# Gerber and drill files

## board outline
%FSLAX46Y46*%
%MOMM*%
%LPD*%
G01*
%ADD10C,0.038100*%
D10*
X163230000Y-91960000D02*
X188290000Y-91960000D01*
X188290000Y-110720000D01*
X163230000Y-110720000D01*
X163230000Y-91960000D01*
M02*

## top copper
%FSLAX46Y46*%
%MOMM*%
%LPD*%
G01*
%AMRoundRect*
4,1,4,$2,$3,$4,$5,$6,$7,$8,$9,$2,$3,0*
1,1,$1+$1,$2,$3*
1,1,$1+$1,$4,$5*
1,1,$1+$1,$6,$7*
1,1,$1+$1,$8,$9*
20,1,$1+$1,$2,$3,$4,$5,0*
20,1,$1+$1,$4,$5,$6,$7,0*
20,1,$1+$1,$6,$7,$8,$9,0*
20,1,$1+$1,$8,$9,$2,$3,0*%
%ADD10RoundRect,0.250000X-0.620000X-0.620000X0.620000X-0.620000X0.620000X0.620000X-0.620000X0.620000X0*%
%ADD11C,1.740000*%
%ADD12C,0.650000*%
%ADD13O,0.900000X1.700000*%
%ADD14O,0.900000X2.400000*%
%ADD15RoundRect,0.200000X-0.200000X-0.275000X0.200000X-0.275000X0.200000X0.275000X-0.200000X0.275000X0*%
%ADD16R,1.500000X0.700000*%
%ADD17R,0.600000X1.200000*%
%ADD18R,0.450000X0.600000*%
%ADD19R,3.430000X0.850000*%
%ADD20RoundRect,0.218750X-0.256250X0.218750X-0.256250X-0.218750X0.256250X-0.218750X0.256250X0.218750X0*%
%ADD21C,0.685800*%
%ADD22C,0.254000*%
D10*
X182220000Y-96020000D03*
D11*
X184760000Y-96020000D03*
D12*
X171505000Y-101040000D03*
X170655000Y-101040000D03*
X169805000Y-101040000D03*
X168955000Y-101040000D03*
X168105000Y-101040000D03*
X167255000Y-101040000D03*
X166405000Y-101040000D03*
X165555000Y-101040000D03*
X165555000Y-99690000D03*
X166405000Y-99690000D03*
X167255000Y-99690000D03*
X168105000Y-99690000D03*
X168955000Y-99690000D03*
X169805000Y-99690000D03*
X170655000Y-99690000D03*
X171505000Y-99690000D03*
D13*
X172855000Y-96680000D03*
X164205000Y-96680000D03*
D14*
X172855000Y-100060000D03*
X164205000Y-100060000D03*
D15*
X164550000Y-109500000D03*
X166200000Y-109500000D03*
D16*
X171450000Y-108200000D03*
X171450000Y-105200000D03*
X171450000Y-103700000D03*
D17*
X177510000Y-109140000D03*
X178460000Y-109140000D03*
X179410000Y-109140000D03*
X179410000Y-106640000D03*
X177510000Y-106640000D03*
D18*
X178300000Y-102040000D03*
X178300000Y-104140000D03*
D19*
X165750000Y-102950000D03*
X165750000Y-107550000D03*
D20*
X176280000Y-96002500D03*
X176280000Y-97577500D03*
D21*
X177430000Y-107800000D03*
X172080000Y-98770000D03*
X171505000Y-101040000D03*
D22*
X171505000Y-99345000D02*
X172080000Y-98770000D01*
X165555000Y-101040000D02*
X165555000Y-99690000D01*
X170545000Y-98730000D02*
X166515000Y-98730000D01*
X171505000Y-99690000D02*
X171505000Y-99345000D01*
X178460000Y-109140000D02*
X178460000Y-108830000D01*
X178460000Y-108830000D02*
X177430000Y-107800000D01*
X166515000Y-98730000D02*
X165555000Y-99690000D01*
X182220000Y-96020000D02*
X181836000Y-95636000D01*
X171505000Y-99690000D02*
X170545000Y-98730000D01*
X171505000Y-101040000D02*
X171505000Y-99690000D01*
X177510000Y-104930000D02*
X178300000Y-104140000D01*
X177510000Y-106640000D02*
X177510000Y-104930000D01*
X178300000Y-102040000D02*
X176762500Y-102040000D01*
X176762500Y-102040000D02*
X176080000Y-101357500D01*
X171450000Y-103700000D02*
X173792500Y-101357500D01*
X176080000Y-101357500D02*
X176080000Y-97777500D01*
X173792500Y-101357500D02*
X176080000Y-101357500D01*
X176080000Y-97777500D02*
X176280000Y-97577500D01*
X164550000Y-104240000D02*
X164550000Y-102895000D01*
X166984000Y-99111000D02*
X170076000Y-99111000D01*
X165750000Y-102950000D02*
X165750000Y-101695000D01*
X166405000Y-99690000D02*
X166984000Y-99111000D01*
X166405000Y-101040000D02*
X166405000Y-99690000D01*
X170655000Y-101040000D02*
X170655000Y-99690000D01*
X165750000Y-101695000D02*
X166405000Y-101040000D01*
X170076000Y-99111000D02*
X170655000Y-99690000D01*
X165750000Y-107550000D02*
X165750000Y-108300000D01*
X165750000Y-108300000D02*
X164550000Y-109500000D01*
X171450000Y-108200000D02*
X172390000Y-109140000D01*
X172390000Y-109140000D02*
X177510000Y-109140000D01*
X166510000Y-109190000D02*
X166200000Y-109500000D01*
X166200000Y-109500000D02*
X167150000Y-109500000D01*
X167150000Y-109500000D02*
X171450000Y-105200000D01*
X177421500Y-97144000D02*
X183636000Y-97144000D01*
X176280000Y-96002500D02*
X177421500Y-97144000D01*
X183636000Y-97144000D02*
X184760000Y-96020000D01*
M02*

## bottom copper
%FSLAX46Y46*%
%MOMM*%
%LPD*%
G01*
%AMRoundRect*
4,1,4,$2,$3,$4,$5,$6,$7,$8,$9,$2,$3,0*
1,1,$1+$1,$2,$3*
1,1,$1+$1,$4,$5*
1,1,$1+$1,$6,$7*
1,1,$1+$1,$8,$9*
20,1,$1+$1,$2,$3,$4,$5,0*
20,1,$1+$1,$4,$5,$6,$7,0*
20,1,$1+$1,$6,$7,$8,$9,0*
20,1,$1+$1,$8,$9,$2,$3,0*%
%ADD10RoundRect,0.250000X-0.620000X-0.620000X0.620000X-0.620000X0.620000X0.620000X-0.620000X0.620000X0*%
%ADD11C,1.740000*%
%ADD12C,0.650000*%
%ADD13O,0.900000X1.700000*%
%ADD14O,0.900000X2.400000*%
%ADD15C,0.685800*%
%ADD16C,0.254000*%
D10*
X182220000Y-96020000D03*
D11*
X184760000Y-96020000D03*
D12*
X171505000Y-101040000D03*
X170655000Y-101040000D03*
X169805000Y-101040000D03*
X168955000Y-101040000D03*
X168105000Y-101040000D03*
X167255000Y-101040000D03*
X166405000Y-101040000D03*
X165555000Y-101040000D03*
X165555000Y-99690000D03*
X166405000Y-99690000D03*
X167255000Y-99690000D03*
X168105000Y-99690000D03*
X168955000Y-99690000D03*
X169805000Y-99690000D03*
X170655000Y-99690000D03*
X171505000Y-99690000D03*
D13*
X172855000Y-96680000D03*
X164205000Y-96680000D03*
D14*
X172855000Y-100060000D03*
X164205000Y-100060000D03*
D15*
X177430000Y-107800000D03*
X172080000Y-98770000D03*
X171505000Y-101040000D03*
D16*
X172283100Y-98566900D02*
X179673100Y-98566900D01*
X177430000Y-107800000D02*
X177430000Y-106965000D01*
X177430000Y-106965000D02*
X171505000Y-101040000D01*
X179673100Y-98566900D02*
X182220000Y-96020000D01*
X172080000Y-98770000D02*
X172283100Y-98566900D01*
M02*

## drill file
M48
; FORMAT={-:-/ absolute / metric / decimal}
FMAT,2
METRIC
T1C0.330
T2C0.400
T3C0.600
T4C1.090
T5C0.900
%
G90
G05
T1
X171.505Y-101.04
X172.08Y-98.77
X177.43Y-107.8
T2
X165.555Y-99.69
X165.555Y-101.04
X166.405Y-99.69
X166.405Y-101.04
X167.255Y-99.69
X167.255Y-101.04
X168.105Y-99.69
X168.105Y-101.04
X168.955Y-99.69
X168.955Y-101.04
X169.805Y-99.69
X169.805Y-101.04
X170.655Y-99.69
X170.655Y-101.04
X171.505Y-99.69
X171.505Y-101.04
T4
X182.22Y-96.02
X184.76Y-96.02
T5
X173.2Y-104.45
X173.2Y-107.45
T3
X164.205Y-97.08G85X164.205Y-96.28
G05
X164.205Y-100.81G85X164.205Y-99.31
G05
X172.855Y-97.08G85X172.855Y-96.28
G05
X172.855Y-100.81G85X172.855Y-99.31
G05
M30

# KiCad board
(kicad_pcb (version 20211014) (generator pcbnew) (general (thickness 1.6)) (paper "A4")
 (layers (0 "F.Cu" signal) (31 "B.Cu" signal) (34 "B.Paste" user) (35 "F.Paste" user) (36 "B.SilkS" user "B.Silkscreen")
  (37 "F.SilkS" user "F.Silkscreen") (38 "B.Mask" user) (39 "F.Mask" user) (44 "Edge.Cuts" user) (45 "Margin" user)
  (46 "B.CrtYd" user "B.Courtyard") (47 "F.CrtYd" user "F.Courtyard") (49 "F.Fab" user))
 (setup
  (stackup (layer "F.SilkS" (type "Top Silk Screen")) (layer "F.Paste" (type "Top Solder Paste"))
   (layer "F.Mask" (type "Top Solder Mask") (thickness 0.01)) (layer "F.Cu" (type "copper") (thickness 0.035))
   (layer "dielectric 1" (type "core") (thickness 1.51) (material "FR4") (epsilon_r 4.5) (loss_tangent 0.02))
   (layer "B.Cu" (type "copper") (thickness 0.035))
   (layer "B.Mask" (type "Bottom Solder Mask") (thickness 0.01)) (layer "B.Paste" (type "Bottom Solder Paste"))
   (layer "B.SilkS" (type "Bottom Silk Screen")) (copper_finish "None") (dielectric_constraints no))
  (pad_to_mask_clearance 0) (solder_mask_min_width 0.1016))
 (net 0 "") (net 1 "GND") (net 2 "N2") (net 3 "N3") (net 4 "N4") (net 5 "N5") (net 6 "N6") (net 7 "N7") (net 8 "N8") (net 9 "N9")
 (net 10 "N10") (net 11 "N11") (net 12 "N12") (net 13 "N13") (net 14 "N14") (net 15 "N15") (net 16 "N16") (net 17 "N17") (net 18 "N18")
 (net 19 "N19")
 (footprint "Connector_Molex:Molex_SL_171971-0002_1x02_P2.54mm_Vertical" (layer "F.Cu") (at 182.22 96.02)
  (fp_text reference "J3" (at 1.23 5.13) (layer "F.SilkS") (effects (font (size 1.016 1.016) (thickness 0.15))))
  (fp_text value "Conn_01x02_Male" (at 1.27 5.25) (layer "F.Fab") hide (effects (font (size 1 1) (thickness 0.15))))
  (pad "1" thru_hole roundrect (at 0 0) (size 1.74 1.74) (drill 1.09) (layers *.Cu *.Mask) (roundrect_rratio 0.143678) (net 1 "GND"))
  (pad "2" thru_hole circle (at 2.54 0) (size 1.74 1.74) (drill 1.09) (layers *.Cu *.Mask) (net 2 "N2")))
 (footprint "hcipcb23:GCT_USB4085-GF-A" (layer "F.Cu") (at 168.53 96.68 180)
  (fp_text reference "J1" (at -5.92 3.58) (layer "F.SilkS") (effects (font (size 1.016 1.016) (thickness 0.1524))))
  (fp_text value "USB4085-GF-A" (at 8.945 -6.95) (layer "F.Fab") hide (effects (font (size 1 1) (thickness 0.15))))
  (pad "A1" thru_hole circle (at -2.975 -4.36 180) (size 0.65 0.65) (drill 0.4) (layers *.Cu *.Mask) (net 1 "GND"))
  (pad "A4" thru_hole circle (at -2.125 -4.36 180) (size 0.65 0.65) (drill 0.4) (layers *.Cu *.Mask) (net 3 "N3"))
  (pad "A5" thru_hole circle (at -1.275 -4.36 180) (size 0.65 0.65) (drill 0.4) (layers *.Cu *.Mask) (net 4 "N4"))
  (pad "A6" thru_hole circle (at -0.425 -4.36 180) (size 0.65 0.65) (drill 0.4) (layers *.Cu *.Mask) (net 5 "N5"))
  (pad "A7" thru_hole circle (at 0.425 -4.36 180) (size 0.65 0.65) (drill 0.4) (layers *.Cu *.Mask) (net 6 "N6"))
  (pad "A8" thru_hole circle (at 1.275 -4.36 180) (size 0.65 0.65) (drill 0.4) (layers *.Cu *.Mask) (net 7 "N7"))
  (pad "A9" thru_hole circle (at 2.125 -4.36 180) (size 0.65 0.65) (drill 0.4) (layers *.Cu *.Mask) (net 3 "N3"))
  (pad "A12" thru_hole circle (at 2.975 -4.36 180) (size 0.65 0.65) (drill 0.4) (layers *.Cu *.Mask) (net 1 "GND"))
  (pad "B1" thru_hole circle (at 2.975 -3.01 180) (size 0.65 0.65) (drill 0.4) (layers *.Cu *.Mask) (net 1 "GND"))
  (pad "B4" thru_hole circle (at 2.125 -3.01 180) (size 0.65 0.65) (drill 0.4) (layers *.Cu *.Mask) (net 3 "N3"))
  (pad "B5" thru_hole circle (at 1.275 -3.01 180) (size 0.65 0.65) (drill 0.4) (layers *.Cu *.Mask) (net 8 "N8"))
  (pad "B6" thru_hole circle (at 0.425 -3.01 180) (size 0.65 0.65) (drill 0.4) (layers *.Cu *.Mask) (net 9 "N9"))
  (pad "B7" thru_hole circle (at -0.425 -3.01 180) (size 0.65 0.65) (drill 0.4) (layers *.Cu *.Mask) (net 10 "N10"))
  (pad "B8" thru_hole circle (at -1.275 -3.01 180) (size 0.65 0.65) (drill 0.4) (layers *.Cu *.Mask) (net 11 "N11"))
  (pad "B9" thru_hole circle (at -2.125 -3.01 180) (size 0.65 0.65) (drill 0.4) (layers *.Cu *.Mask) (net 3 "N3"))
  (pad "B12" thru_hole circle (at -2.975 -3.01 180) (size 0.65 0.65) (drill 0.4) (layers *.Cu *.Mask) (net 1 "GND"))
  (pad "S1" thru_hole oval (at -4.325 0 180) (size 0.9 1.7) (drill oval 0.6 1.4) (layers *.Cu *.Mask) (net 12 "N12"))
  (pad "S2" thru_hole oval (at 4.325 0 180) (size 0.9 1.7) (drill oval 0.6 1.4) (layers *.Cu *.Mask) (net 12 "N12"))
  (pad "S3" thru_hole oval (at -4.325 -3.38 180) (size 0.9 2.4) (drill oval 0.6 2.1) (layers *.Cu *.Mask) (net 12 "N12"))
  (pad "S4" thru_hole oval (at 4.325 -3.38 180) (size 0.9 2.4) (drill oval 0.6 2.1) (layers *.Cu *.Mask) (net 12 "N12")))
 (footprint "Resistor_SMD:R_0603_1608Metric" (layer "F.Cu") (at 165.375 109.5)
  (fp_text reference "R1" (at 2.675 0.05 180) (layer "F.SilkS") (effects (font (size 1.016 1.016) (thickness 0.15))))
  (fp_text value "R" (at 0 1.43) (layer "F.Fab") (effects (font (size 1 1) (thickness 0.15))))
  (pad "1" smd roundrect (at -0.825 0) (size 0.8 0.95) (layers "F.Cu" "F.Paste" "F.Mask") (roundrect_rratio 0.25) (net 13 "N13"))
  (pad "2" smd roundrect (at 0.825 0) (size 0.8 0.95) (layers "F.Cu" "F.Paste" "F.Mask") (roundrect_rratio 0.25) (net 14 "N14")))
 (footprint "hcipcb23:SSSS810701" (layer "F.Cu") (at 171.45 105.2 90)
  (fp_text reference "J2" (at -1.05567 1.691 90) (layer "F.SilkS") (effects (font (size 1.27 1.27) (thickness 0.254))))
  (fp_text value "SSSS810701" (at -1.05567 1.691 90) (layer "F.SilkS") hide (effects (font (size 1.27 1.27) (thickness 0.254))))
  (pad "" np_thru_hole circle (at 0.75 1.75 90) (size 0.9 0.9) (drill 0.9) (layers *.Cu *.Mask))
  (pad "" np_thru_hole circle (at -2.25 1.75 90) (size 0.9 0.9) (drill 0.9) (layers *.Cu *.Mask))
  (pad "1" smd rect (at -3 0 90) (size 0.7 1.5) (layers "F.Cu" "F.Paste" "F.Mask") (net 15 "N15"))
  (pad "2" smd rect (at 0 0 90) (size 0.7 1.5) (layers "F.Cu" "F.Paste" "F.Mask") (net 14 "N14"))
  (pad "3" smd rect (at 1.5 0 90) (size 0.7 1.5) (layers "F.Cu" "F.Paste" "F.Mask") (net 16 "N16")))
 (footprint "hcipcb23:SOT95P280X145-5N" (layer "F.Cu") (at 178.46 107.89 90)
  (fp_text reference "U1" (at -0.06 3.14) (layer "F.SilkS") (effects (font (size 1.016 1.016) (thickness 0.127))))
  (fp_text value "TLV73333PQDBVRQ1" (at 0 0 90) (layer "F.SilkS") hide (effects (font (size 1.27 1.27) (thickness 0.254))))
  (pad "1" smd rect (at -1.25 -0.95 180) (size 0.6 1.2) (layers "F.Cu" "F.Paste" "F.Mask") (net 15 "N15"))
  (pad "2" smd rect (at -1.25 0 180) (size 0.6 1.2) (layers "F.Cu" "F.Paste" "F.Mask") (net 1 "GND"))
  (pad "3" smd rect (at -1.25 0.95 180) (size 0.6 1.2) (layers "F.Cu" "F.Paste" "F.Mask") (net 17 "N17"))
  (pad "4" smd rect (at 1.25 0.95 180) (size 0.6 1.2) (layers "F.Cu" "F.Paste" "F.Mask") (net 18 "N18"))
  (pad "5" smd rect (at 1.25 -0.95 180) (size 0.6 1.2) (layers "F.Cu" "F.Paste" "F.Mask") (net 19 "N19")))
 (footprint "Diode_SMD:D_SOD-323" (layer "F.Cu") (at 178.3 103.09 -90)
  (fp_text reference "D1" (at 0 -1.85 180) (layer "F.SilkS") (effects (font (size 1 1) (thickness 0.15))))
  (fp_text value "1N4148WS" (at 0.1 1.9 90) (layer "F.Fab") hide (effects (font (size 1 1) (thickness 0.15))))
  (pad "1" smd rect (at -1.05 0 270) (size 0.6 0.45) (layers "F.Cu" "F.Paste" "F.Mask") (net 16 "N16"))
  (pad "2" smd rect (at 1.05 0 270) (size 0.6 0.45) (layers "F.Cu" "F.Paste" "F.Mask") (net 19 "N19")))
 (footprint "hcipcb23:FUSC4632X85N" (layer "F.Cu") (at 165.75 105.25 -90)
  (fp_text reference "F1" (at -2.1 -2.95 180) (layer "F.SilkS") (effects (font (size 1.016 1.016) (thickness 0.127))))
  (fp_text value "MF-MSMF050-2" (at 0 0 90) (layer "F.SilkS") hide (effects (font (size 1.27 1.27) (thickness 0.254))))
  (pad "1" smd rect (at -2.3 0 270) (size 0.85 3.43) (layers "F.Cu" "F.Paste" "F.Mask") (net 3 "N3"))
  (pad "2" smd rect (at 2.3 0 270) (size 0.85 3.43) (layers "F.Cu" "F.Paste" "F.Mask") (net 13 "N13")))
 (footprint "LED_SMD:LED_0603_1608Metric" (layer "F.Cu") (at 176.28 96.79 -90)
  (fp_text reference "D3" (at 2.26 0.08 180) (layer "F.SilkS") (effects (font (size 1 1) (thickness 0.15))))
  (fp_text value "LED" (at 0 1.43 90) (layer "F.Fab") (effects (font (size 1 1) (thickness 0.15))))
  (pad "1" smd roundrect (at -0.7875 0 270) (size 0.875 0.95) (layers "F.Cu" "F.Paste" "F.Mask") (roundrect_rratio 0.25) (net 2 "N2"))
  (pad "2" smd roundrect (at 0.7875 0 270) (size 0.875 0.95) (layers "F.Cu" "F.Paste" "F.Mask") (roundrect_rratio 0.25) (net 16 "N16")))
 (gr_rect (start 163.23 91.96) (end 188.29 110.72) (layer "Edge.Cuts") (width 0.0381) (fill none))
 (segment (start 171.505 99.345) (end 172.08 98.77) (width 0.254) (layer "F.Cu") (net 1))
 (segment (start 165.555 101.04) (end 165.555 99.69) (width 0.254) (layer "F.Cu") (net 1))
 (segment (start 170.545 98.73) (end 166.515 98.73) (width 0.254) (layer "F.Cu") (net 1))
 (segment (start 171.505 99.69) (end 171.505 99.345) (width 0.254) (layer "F.Cu") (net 1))
 (segment (start 178.46 109.14) (end 178.46 108.83) (width 0.254) (layer "F.Cu") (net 1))
 (segment (start 178.46 108.83) (end 177.43 107.8) (width 0.254) (layer "F.Cu") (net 1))
 (segment (start 166.515 98.73) (end 165.555 99.69) (width 0.254) (layer "F.Cu") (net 1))
 (segment (start 182.22 96.02) (end 181.836 95.636) (width 0.254) (layer "F.Cu") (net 1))
 (segment (start 171.505 99.69) (end 170.545 98.73) (width 0.254) (layer "F.Cu") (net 1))
 (segment (start 171.505 101.04) (end 171.505 99.69) (width 0.254) (layer "F.Cu") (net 1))
 (via (at 177.43 107.8) (size 0.6858) (drill 0.3302) (layers "F.Cu" "B.Cu") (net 1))
 (via (at 172.08 98.77) (size 0.6858) (drill 0.3302) (layers "F.Cu" "B.Cu") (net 1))
 (via (at 171.505 101.04) (size 0.6858) (drill 0.3302) (layers "F.Cu" "B.Cu") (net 1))
 (segment (start 172.2831 98.5669) (end 179.6731 98.5669) (width 0.254) (layer "B.Cu") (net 1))
 (segment (start 177.43 107.8) (end 177.43 106.965) (width 0.254) (layer "B.Cu") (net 1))
 (segment (start 177.43 106.965) (end 171.505 101.04) (width 0.254) (layer "B.Cu") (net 1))
 (segment (start 179.6731 98.5669) (end 182.22 96.02) (width 0.254) (layer "B.Cu") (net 1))
 (segment (start 172.08 98.77) (end 172.2831 98.5669) (width 0.254) (layer "B.Cu") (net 1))
 (segment (start 177.51 104.93) (end 178.3 104.14) (width 0.254) (layer "F.Cu") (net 19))
 (segment (start 177.51 106.64) (end 177.51 104.93) (width 0.254) (layer "F.Cu") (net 19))
 (segment (start 178.3 102.04) (end 176.7625 102.04) (width 0.254) (layer "F.Cu") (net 16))
 (segment (start 176.7625 102.04) (end 176.08 101.3575) (width 0.254) (layer "F.Cu") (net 16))
 (segment (start 171.45 103.7) (end 173.7925 101.3575) (width 0.254) (layer "F.Cu") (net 16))
 (segment (start 176.08 101.3575) (end 176.08 97.7775) (width 0.254) (layer "F.Cu") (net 16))
 (segment (start 173.7925 101.3575) (end 176.08 101.3575) (width 0.254) (layer "F.Cu") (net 16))
 (segment (start 176.08 97.7775) (end 176.28 97.5775) (width 0.254) (layer "F.Cu") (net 16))
 (segment (start 164.55 104.24) (end 164.55 102.895) (width 0.254) (layer "F.Cu") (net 3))
 (segment (start 166.984 99.111) (end 170.076 99.111) (width 0.254) (layer "F.Cu") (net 3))
 (segment (start 165.75 102.95) (end 165.75 101.695) (width 0.254) (layer "F.Cu") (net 3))
 (segment (start 166.405 99.69) (end 166.984 99.111) (width 0.254) (layer "F.Cu") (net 3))
 (segment (start 166.405 101.04) (end 166.405 99.69) (width 0.254) (layer "F.Cu") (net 3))
 (segment (start 170.655 101.04) (end 170.655 99.69) (width 0.254) (layer "F.Cu") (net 3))
 (segment (start 165.75 101.695) (end 166.405 101.04) (width 0.254) (layer "F.Cu") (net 3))
 (segment (start 170.076 99.111) (end 170.655 99.69) (width 0.254) (layer "F.Cu") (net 3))
 (segment (start 165.75 107.55) (end 165.75 108.3) (width 0.254) (layer "F.Cu") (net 13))
 (segment (start 165.75 108.3) (end 164.55 109.5) (width 0.254) (layer "F.Cu") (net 13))
 (segment (start 171.45 108.2) (end 172.39 109.14) (width 0.254) (layer "F.Cu") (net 15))
 (segment (start 172.39 109.14) (end 177.51 109.14) (width 0.254) (layer "F.Cu") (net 15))
 (segment (start 166.51 109.19) (end 166.2 109.5) (width 0.254) (layer "F.Cu") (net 14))
 (segment (start 166.2 109.5) (end 167.15 109.5) (width 0.254) (layer "F.Cu") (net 14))
 (segment (start 167.15 109.5) (end 171.45 105.2) (width 0.254) (layer "F.Cu") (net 14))
 (segment (start 177.4215 97.144) (end 183.636 97.144) (width 0.254) (layer "F.Cu") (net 2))
 (segment (start 176.28 96.0025) (end 177.4215 97.144) (width 0.254) (layer "F.Cu") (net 2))
 (segment (start 183.636 97.144) (end 184.76 96.02) (width 0.254) (layer "F.Cu") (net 2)))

